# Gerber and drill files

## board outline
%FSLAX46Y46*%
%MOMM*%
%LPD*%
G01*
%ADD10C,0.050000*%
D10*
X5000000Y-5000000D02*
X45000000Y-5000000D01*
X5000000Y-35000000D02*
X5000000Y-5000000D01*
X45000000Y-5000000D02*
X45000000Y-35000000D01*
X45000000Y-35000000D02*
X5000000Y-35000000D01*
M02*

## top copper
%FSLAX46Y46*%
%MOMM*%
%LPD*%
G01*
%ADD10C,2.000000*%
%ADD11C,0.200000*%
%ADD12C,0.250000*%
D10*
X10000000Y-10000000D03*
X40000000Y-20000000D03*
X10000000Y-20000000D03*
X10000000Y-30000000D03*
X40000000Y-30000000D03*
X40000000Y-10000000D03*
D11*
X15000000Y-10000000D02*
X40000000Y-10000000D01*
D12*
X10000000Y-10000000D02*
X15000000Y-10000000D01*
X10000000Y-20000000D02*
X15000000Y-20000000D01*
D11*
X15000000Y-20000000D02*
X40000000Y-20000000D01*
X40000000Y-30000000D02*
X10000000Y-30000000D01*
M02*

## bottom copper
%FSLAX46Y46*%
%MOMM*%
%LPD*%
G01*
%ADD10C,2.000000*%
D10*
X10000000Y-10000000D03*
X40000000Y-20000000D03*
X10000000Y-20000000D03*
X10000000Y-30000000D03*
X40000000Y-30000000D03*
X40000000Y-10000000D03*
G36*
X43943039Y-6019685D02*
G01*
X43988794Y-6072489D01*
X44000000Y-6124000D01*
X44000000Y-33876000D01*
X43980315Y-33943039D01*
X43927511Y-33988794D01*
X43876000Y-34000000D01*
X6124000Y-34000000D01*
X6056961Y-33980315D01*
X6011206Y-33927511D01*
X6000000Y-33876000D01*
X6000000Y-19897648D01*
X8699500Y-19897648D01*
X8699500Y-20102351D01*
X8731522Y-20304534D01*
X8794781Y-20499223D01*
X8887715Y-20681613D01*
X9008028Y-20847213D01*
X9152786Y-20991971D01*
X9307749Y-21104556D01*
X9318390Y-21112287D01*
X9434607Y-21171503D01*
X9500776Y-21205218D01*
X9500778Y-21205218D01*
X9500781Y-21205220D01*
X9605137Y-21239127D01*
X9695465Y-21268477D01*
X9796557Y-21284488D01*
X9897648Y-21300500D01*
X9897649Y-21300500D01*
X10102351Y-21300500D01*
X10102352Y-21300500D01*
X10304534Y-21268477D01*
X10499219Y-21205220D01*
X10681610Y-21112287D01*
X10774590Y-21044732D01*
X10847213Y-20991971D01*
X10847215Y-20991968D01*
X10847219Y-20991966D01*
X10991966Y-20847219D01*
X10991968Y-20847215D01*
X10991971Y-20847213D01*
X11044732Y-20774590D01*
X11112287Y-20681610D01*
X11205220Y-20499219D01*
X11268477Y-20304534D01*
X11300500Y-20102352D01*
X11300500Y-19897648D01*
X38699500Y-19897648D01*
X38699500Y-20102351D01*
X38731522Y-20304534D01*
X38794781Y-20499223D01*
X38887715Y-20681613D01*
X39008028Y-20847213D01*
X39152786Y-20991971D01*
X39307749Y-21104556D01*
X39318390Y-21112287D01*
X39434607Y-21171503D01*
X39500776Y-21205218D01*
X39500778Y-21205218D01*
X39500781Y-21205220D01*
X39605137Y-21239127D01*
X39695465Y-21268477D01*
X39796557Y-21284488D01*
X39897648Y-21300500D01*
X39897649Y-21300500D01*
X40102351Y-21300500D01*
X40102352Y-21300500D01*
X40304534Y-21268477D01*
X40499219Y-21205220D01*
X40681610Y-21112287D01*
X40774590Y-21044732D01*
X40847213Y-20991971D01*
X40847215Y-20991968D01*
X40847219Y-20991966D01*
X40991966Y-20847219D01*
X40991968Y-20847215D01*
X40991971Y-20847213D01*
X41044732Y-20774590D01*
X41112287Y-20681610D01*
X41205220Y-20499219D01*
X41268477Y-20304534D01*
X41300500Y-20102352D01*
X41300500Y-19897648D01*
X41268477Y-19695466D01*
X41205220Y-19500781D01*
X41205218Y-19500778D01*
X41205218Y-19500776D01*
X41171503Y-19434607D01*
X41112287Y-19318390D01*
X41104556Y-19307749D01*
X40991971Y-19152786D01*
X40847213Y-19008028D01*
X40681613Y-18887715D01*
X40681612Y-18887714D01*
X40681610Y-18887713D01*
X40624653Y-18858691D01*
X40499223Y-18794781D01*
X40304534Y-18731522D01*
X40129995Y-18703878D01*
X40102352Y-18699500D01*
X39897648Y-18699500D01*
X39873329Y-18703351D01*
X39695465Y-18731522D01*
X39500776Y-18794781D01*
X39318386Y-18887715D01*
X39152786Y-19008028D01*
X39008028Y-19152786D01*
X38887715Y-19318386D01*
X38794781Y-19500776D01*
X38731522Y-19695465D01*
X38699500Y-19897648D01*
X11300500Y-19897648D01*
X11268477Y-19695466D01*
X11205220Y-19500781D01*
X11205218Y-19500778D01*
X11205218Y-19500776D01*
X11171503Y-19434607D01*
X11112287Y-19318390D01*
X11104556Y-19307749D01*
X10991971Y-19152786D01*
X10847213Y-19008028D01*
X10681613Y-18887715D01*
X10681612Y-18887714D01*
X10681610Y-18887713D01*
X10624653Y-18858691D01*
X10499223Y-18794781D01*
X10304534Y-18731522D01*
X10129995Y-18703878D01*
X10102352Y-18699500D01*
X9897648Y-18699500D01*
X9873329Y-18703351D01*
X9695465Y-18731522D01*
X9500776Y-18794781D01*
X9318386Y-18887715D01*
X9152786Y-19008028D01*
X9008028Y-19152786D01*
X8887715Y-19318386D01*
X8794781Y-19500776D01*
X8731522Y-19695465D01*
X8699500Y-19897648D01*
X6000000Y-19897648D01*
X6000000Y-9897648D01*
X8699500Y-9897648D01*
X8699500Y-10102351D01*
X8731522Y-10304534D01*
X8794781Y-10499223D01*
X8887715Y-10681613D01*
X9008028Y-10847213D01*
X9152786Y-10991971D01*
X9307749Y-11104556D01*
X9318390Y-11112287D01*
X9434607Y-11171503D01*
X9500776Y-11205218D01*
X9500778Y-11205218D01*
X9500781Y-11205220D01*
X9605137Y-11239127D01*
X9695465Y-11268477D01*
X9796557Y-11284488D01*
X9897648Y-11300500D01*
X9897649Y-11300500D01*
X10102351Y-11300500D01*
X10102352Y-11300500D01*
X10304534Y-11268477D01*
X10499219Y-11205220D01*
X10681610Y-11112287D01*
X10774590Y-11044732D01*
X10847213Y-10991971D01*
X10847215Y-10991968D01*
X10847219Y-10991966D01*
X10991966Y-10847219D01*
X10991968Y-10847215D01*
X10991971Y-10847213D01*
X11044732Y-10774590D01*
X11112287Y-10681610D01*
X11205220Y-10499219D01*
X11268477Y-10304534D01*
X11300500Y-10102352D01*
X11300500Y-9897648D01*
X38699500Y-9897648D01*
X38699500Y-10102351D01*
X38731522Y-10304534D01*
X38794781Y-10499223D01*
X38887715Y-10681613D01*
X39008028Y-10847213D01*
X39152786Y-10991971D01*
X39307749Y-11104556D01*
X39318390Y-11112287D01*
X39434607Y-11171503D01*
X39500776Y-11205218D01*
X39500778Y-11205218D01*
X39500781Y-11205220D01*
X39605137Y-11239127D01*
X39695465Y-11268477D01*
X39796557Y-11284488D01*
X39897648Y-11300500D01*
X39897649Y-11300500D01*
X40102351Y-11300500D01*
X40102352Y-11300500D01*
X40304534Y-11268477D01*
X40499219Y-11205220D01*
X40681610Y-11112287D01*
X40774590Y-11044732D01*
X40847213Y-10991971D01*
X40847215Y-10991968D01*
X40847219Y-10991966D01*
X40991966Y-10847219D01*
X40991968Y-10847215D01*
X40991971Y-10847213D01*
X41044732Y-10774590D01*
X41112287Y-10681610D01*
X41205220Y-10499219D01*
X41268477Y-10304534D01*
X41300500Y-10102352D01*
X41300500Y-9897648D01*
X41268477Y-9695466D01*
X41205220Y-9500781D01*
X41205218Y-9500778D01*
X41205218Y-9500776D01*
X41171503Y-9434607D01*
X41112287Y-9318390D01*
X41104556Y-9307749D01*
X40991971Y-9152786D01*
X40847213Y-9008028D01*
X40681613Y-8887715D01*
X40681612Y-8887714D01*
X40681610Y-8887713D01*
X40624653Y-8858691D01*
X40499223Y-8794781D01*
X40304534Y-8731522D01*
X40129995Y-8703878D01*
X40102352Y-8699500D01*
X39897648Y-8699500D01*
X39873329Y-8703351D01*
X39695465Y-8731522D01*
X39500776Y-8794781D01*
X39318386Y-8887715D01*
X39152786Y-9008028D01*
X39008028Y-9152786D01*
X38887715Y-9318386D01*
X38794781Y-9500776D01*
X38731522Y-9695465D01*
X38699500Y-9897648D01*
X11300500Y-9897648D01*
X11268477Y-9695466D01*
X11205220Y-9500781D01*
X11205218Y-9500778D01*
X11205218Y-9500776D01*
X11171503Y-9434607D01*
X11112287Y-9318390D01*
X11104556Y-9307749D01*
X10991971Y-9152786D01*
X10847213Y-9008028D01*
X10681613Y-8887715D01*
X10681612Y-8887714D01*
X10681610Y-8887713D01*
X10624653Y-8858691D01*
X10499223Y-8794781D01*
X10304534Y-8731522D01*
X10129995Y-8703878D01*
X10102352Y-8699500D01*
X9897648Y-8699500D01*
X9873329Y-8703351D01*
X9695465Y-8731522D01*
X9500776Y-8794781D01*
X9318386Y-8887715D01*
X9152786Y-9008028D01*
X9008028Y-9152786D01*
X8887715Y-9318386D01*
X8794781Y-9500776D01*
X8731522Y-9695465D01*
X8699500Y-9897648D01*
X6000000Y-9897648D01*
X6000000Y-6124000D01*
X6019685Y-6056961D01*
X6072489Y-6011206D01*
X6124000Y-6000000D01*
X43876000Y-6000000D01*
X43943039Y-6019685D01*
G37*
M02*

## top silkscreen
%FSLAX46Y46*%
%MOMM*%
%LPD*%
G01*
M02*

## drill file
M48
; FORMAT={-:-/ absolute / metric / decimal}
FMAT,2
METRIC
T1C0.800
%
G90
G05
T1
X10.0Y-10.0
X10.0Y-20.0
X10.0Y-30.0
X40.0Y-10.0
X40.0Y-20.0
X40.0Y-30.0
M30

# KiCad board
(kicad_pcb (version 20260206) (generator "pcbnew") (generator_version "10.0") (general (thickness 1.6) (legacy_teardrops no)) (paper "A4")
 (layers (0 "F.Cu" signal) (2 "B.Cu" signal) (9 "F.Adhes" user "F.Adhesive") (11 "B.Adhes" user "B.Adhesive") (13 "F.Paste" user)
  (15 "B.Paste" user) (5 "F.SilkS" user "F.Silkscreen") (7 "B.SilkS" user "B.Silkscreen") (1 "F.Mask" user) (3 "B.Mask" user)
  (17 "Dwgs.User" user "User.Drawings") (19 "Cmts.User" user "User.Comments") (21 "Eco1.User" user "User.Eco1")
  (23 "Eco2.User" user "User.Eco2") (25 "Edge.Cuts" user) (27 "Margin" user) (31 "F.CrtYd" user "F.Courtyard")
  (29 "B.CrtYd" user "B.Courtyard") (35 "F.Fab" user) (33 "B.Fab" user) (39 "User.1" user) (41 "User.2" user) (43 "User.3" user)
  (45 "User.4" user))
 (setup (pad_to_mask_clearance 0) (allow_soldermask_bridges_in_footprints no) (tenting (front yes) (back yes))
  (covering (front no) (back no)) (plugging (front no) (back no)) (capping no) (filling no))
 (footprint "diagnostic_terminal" (layer "F.Cu") (at 10 10)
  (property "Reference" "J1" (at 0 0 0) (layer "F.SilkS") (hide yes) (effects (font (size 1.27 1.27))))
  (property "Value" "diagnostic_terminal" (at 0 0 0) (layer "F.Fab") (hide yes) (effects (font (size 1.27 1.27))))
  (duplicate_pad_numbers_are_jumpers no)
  (pad "1" thru_hole circle (at 0 0) (size 2 2) (drill 0.8) (layers "*.Cu") (remove_unused_layers no) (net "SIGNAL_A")))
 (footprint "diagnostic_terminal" (layer "F.Cu") (at 40 20)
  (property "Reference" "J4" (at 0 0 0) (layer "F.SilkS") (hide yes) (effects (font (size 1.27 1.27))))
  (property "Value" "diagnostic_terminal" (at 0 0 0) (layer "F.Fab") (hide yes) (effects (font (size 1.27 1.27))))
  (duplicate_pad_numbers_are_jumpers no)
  (pad "1" thru_hole circle (at 0 0) (size 2 2) (drill 0.8) (layers "*.Cu") (remove_unused_layers no) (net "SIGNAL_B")))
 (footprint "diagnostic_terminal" (layer "F.Cu") (at 10 20)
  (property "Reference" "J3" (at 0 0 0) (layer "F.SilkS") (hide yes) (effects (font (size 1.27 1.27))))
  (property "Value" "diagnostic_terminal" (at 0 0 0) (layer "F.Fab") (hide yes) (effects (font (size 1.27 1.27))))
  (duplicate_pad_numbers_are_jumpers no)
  (pad "1" thru_hole circle (at 0 0) (size 2 2) (drill 0.8) (layers "*.Cu") (remove_unused_layers no) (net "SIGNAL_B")))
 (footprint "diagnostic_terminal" (layer "F.Cu") (at 10 30)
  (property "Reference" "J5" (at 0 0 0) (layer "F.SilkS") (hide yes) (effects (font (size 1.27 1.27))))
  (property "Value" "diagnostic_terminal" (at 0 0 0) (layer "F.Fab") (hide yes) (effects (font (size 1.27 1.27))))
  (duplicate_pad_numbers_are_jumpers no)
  (pad "1" thru_hole circle (at 0 0) (size 2 2) (drill 0.8) (layers "*.Cu") (remove_unused_layers no) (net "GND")))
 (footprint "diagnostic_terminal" (layer "F.Cu") (at 40 30)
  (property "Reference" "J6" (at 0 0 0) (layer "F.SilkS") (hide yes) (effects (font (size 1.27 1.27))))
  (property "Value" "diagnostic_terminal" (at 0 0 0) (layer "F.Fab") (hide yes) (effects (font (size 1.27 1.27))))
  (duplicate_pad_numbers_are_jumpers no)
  (pad "1" thru_hole circle (at 0 0) (size 2 2) (drill 0.8) (layers "*.Cu") (remove_unused_layers no) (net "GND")))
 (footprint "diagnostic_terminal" (layer "F.Cu") (at 40 10)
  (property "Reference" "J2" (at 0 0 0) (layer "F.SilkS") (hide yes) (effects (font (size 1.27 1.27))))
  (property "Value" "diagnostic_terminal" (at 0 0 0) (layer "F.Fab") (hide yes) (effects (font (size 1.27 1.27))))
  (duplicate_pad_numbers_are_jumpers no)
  (pad "1" thru_hole circle (at 0 0) (size 2 2) (drill 0.8) (layers "*.Cu") (remove_unused_layers no) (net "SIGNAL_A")))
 (gr_line (start 5 5) (end 45 5) (stroke (width 0.05) (type default)) (layer "Edge.Cuts"))
 (gr_line (start 5 35) (end 5 5) (stroke (width 0.05) (type default)) (layer "Edge.Cuts"))
 (gr_line (start 45 5) (end 45 35) (stroke (width 0.05) (type default)) (layer "Edge.Cuts"))
 (gr_line (start 45 35) (end 5 35) (stroke (width 0.05) (type default)) (layer "Edge.Cuts"))
 (segment (start 15 10) (end 40 10) (width 0.2) (layer "F.Cu") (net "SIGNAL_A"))
 (segment (start 10 10) (end 15 10) (width 0.25) (layer "F.Cu") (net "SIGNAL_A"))
 (segment (start 10 20) (end 15 20) (width 0.25) (layer "F.Cu") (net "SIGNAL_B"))
 (segment (start 15 20) (end 40 20) (width 0.2) (layer "F.Cu") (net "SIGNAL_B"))
 (segment (start 40 30) (end 10 30) (width 0.2) (layer "F.Cu") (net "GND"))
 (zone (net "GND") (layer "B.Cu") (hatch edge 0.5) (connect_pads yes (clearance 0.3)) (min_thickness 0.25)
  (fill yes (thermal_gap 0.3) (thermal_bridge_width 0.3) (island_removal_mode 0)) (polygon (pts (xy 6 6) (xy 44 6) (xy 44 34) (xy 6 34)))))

